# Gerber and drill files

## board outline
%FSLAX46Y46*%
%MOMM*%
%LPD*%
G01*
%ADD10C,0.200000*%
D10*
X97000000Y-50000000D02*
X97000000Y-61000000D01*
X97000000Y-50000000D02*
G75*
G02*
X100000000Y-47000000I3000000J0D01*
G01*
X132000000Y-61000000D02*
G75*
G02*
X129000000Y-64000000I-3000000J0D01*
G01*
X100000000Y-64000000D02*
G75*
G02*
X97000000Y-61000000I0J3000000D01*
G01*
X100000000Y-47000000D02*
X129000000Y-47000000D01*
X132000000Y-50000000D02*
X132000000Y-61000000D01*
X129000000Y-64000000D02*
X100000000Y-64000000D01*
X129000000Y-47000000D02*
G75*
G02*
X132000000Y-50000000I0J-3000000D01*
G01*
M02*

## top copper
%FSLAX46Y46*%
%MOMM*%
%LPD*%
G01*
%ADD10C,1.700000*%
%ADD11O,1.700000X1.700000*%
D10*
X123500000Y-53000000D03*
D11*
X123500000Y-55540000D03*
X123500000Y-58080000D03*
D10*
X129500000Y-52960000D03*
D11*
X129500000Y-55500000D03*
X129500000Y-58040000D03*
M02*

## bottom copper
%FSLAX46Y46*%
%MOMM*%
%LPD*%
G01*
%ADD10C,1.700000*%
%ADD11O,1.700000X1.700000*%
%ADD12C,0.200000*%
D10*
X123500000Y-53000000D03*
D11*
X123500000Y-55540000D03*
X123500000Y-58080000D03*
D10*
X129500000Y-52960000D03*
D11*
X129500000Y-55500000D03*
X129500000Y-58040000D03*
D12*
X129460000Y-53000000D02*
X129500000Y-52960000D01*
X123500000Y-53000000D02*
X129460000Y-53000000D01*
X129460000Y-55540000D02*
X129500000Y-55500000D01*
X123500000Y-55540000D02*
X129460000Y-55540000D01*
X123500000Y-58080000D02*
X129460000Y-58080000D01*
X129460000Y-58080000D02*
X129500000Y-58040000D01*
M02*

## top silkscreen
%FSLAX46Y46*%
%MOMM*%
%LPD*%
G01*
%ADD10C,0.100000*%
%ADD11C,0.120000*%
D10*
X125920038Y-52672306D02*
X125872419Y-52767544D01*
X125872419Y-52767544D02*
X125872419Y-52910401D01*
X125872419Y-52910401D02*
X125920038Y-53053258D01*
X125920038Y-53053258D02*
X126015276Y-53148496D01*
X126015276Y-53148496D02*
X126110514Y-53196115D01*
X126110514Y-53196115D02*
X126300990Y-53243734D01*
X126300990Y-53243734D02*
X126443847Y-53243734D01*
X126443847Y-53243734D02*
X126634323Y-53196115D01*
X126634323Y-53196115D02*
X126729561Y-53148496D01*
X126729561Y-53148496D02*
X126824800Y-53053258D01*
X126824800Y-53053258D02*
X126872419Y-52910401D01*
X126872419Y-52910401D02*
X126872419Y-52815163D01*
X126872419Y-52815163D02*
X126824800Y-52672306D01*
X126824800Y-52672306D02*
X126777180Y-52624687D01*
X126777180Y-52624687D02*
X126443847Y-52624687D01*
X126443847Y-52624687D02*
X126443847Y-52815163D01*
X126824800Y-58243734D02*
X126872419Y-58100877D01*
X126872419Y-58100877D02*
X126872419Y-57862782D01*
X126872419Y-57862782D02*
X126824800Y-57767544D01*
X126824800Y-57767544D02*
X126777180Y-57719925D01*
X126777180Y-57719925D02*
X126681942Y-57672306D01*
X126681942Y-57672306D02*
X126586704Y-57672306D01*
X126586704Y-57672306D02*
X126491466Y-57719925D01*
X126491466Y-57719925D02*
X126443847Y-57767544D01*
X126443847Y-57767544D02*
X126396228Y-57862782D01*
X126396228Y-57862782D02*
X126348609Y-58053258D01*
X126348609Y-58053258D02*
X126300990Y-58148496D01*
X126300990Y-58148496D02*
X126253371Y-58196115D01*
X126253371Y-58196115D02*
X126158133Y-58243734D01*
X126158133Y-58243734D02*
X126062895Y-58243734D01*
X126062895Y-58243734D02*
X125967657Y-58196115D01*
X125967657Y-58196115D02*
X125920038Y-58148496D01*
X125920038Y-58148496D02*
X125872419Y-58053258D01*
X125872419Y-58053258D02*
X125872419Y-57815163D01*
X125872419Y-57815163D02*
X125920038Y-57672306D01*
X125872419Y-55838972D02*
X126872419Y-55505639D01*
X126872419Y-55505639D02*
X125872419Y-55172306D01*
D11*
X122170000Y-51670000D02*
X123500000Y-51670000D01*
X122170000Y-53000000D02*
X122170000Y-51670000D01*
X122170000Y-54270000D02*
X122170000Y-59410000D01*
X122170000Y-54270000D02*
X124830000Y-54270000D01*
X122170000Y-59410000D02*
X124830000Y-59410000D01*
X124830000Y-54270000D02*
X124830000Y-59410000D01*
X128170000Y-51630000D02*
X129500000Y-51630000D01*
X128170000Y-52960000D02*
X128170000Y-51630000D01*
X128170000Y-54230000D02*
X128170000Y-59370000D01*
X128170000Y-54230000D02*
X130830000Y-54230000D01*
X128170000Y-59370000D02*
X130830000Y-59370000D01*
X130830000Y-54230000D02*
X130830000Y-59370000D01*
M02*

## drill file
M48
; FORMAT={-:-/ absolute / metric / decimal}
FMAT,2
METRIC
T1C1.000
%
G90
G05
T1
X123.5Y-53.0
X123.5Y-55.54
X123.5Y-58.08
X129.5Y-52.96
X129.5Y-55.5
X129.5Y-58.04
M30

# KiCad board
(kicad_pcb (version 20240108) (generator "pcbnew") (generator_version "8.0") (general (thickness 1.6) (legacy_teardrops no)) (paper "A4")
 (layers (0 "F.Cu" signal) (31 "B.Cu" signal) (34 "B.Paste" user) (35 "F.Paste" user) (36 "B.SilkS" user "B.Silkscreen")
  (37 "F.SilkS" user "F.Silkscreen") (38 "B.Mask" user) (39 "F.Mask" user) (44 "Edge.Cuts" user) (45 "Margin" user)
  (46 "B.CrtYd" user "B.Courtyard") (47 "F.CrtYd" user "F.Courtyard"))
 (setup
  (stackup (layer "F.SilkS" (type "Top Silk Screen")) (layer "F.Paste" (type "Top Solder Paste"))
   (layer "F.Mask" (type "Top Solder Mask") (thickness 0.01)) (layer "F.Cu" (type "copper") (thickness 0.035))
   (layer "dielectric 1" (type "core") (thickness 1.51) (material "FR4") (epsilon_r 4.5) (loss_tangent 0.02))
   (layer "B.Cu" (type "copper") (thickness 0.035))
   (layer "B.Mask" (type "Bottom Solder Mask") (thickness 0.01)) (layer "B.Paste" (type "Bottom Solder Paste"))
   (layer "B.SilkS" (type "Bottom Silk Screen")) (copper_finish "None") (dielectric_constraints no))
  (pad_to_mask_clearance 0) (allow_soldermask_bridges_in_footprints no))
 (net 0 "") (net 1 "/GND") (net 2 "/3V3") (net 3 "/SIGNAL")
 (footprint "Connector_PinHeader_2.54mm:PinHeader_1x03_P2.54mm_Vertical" (layer "F.Cu") (at 123.5 53)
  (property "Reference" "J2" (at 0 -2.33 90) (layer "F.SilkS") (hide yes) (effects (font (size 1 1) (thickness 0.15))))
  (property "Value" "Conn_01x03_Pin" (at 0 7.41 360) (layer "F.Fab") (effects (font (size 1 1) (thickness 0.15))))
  (fp_line (start -1.33 -1.33) (end 0 -1.33) (stroke (width 0.12) (type solid)) (layer "F.SilkS"))
  (fp_line (start -1.33 0) (end -1.33 -1.33) (stroke (width 0.12) (type solid)) (layer "F.SilkS"))
  (fp_line (start -1.33 1.27) (end -1.33 6.41) (stroke (width 0.12) (type solid)) (layer "F.SilkS"))
  (fp_line (start -1.33 1.27) (end 1.33 1.27) (stroke (width 0.12) (type solid)) (layer "F.SilkS"))
  (fp_line (start -1.33 6.41) (end 1.33 6.41) (stroke (width 0.12) (type solid)) (layer "F.SilkS"))
  (fp_line (start 1.33 1.27) (end 1.33 6.41) (stroke (width 0.12) (type solid)) (layer "F.SilkS"))
  (pad "1" thru_hole circle (at 0 0) (size 1.7 1.7) (drill 1) (layers "*.Cu" "*.Mask") (remove_unused_layers no) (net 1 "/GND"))
  (pad "2" thru_hole oval (at 0 2.54) (size 1.7 1.7) (drill 1) (layers "*.Cu" "*.Mask") (remove_unused_layers no) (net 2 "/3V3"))
  (pad "3" thru_hole oval (at 0 5.08) (size 1.7 1.7) (drill 1) (layers "*.Cu" "*.Mask") (remove_unused_layers no) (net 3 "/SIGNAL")))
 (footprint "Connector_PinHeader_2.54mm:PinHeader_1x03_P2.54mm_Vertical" (layer "F.Cu") (at 129.5 52.96)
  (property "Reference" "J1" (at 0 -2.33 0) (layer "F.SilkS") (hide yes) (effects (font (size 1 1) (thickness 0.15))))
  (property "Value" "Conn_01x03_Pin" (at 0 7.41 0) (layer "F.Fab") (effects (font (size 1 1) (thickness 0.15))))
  (fp_line (start -1.33 -1.33) (end 0 -1.33) (stroke (width 0.12) (type solid)) (layer "F.SilkS"))
  (fp_line (start -1.33 0) (end -1.33 -1.33) (stroke (width 0.12) (type solid)) (layer "F.SilkS"))
  (fp_line (start -1.33 1.27) (end -1.33 6.41) (stroke (width 0.12) (type solid)) (layer "F.SilkS"))
  (fp_line (start -1.33 1.27) (end 1.33 1.27) (stroke (width 0.12) (type solid)) (layer "F.SilkS"))
  (fp_line (start -1.33 6.41) (end 1.33 6.41) (stroke (width 0.12) (type solid)) (layer "F.SilkS"))
  (fp_line (start 1.33 1.27) (end 1.33 6.41) (stroke (width 0.12) (type solid)) (layer "F.SilkS"))
  (pad "1" thru_hole circle (at 0 0) (size 1.7 1.7) (drill 1) (layers "*.Cu" "*.Mask") (remove_unused_layers no) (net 1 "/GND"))
  (pad "2" thru_hole oval (at 0 2.54) (size 1.7 1.7) (drill 1) (layers "*.Cu" "*.Mask") (remove_unused_layers no) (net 2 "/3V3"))
  (pad "3" thru_hole oval (at 0 5.08) (size 1.7 1.7) (drill 1) (layers "*.Cu" "*.Mask") (remove_unused_layers no) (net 3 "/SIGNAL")))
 (gr_line (start 97 50) (end 97 61) (locked yes) (stroke (width 0.2) (type default)) (layer "Edge.Cuts"))
 (gr_arc (start 97 50) (mid 97.87868 47.87868) (end 100 47) (locked yes) (stroke (width 0.2) (type default)) (layer "Edge.Cuts"))
 (gr_arc (start 132 61) (mid 131.12132 63.12132) (end 129 64) (locked yes) (stroke (width 0.2) (type default)) (layer "Edge.Cuts"))
 (gr_arc (start 100 64) (mid 97.87868 63.12132) (end 97 61) (locked yes) (stroke (width 0.2) (type default)) (layer "Edge.Cuts"))
 (gr_line (start 100 47) (end 129 47) (locked yes) (stroke (width 0.2) (type default)) (layer "Edge.Cuts"))
 (gr_line (start 132 50) (end 132 61) (locked yes) (stroke (width 0.2) (type default)) (layer "Edge.Cuts"))
 (gr_line (start 129 64) (end 100 64) (locked yes) (stroke (width 0.2) (type default)) (layer "Edge.Cuts"))
 (gr_arc (start 129 47) (mid 131.12132 47.87868) (end 132 50) (locked yes) (stroke (width 0.2) (type default)) (layer "Edge.Cuts"))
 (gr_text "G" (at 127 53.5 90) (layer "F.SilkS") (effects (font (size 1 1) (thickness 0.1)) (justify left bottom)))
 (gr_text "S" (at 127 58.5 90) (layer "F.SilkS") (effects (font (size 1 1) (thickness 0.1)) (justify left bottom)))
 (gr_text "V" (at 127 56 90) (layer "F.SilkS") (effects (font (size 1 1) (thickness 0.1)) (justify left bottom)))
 (segment (start 129.46 53) (end 129.5 52.96) (width 0.2) (layer "B.Cu") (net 1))
 (segment (start 123.5 53) (end 129.46 53) (width 0.2) (layer "B.Cu") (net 1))
 (segment (start 129.46 55.54) (end 129.5 55.5) (width 0.2) (layer "B.Cu") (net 2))
 (segment (start 123.5 55.54) (end 129.46 55.54) (width 0.2) (layer "B.Cu") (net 2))
 (segment (start 123.5 58.08) (end 129.46 58.08) (width 0.2) (layer "B.Cu") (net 3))
 (segment (start 129.46 58.08) (end 129.5 58.04) (width 0.2) (layer "B.Cu") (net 3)))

